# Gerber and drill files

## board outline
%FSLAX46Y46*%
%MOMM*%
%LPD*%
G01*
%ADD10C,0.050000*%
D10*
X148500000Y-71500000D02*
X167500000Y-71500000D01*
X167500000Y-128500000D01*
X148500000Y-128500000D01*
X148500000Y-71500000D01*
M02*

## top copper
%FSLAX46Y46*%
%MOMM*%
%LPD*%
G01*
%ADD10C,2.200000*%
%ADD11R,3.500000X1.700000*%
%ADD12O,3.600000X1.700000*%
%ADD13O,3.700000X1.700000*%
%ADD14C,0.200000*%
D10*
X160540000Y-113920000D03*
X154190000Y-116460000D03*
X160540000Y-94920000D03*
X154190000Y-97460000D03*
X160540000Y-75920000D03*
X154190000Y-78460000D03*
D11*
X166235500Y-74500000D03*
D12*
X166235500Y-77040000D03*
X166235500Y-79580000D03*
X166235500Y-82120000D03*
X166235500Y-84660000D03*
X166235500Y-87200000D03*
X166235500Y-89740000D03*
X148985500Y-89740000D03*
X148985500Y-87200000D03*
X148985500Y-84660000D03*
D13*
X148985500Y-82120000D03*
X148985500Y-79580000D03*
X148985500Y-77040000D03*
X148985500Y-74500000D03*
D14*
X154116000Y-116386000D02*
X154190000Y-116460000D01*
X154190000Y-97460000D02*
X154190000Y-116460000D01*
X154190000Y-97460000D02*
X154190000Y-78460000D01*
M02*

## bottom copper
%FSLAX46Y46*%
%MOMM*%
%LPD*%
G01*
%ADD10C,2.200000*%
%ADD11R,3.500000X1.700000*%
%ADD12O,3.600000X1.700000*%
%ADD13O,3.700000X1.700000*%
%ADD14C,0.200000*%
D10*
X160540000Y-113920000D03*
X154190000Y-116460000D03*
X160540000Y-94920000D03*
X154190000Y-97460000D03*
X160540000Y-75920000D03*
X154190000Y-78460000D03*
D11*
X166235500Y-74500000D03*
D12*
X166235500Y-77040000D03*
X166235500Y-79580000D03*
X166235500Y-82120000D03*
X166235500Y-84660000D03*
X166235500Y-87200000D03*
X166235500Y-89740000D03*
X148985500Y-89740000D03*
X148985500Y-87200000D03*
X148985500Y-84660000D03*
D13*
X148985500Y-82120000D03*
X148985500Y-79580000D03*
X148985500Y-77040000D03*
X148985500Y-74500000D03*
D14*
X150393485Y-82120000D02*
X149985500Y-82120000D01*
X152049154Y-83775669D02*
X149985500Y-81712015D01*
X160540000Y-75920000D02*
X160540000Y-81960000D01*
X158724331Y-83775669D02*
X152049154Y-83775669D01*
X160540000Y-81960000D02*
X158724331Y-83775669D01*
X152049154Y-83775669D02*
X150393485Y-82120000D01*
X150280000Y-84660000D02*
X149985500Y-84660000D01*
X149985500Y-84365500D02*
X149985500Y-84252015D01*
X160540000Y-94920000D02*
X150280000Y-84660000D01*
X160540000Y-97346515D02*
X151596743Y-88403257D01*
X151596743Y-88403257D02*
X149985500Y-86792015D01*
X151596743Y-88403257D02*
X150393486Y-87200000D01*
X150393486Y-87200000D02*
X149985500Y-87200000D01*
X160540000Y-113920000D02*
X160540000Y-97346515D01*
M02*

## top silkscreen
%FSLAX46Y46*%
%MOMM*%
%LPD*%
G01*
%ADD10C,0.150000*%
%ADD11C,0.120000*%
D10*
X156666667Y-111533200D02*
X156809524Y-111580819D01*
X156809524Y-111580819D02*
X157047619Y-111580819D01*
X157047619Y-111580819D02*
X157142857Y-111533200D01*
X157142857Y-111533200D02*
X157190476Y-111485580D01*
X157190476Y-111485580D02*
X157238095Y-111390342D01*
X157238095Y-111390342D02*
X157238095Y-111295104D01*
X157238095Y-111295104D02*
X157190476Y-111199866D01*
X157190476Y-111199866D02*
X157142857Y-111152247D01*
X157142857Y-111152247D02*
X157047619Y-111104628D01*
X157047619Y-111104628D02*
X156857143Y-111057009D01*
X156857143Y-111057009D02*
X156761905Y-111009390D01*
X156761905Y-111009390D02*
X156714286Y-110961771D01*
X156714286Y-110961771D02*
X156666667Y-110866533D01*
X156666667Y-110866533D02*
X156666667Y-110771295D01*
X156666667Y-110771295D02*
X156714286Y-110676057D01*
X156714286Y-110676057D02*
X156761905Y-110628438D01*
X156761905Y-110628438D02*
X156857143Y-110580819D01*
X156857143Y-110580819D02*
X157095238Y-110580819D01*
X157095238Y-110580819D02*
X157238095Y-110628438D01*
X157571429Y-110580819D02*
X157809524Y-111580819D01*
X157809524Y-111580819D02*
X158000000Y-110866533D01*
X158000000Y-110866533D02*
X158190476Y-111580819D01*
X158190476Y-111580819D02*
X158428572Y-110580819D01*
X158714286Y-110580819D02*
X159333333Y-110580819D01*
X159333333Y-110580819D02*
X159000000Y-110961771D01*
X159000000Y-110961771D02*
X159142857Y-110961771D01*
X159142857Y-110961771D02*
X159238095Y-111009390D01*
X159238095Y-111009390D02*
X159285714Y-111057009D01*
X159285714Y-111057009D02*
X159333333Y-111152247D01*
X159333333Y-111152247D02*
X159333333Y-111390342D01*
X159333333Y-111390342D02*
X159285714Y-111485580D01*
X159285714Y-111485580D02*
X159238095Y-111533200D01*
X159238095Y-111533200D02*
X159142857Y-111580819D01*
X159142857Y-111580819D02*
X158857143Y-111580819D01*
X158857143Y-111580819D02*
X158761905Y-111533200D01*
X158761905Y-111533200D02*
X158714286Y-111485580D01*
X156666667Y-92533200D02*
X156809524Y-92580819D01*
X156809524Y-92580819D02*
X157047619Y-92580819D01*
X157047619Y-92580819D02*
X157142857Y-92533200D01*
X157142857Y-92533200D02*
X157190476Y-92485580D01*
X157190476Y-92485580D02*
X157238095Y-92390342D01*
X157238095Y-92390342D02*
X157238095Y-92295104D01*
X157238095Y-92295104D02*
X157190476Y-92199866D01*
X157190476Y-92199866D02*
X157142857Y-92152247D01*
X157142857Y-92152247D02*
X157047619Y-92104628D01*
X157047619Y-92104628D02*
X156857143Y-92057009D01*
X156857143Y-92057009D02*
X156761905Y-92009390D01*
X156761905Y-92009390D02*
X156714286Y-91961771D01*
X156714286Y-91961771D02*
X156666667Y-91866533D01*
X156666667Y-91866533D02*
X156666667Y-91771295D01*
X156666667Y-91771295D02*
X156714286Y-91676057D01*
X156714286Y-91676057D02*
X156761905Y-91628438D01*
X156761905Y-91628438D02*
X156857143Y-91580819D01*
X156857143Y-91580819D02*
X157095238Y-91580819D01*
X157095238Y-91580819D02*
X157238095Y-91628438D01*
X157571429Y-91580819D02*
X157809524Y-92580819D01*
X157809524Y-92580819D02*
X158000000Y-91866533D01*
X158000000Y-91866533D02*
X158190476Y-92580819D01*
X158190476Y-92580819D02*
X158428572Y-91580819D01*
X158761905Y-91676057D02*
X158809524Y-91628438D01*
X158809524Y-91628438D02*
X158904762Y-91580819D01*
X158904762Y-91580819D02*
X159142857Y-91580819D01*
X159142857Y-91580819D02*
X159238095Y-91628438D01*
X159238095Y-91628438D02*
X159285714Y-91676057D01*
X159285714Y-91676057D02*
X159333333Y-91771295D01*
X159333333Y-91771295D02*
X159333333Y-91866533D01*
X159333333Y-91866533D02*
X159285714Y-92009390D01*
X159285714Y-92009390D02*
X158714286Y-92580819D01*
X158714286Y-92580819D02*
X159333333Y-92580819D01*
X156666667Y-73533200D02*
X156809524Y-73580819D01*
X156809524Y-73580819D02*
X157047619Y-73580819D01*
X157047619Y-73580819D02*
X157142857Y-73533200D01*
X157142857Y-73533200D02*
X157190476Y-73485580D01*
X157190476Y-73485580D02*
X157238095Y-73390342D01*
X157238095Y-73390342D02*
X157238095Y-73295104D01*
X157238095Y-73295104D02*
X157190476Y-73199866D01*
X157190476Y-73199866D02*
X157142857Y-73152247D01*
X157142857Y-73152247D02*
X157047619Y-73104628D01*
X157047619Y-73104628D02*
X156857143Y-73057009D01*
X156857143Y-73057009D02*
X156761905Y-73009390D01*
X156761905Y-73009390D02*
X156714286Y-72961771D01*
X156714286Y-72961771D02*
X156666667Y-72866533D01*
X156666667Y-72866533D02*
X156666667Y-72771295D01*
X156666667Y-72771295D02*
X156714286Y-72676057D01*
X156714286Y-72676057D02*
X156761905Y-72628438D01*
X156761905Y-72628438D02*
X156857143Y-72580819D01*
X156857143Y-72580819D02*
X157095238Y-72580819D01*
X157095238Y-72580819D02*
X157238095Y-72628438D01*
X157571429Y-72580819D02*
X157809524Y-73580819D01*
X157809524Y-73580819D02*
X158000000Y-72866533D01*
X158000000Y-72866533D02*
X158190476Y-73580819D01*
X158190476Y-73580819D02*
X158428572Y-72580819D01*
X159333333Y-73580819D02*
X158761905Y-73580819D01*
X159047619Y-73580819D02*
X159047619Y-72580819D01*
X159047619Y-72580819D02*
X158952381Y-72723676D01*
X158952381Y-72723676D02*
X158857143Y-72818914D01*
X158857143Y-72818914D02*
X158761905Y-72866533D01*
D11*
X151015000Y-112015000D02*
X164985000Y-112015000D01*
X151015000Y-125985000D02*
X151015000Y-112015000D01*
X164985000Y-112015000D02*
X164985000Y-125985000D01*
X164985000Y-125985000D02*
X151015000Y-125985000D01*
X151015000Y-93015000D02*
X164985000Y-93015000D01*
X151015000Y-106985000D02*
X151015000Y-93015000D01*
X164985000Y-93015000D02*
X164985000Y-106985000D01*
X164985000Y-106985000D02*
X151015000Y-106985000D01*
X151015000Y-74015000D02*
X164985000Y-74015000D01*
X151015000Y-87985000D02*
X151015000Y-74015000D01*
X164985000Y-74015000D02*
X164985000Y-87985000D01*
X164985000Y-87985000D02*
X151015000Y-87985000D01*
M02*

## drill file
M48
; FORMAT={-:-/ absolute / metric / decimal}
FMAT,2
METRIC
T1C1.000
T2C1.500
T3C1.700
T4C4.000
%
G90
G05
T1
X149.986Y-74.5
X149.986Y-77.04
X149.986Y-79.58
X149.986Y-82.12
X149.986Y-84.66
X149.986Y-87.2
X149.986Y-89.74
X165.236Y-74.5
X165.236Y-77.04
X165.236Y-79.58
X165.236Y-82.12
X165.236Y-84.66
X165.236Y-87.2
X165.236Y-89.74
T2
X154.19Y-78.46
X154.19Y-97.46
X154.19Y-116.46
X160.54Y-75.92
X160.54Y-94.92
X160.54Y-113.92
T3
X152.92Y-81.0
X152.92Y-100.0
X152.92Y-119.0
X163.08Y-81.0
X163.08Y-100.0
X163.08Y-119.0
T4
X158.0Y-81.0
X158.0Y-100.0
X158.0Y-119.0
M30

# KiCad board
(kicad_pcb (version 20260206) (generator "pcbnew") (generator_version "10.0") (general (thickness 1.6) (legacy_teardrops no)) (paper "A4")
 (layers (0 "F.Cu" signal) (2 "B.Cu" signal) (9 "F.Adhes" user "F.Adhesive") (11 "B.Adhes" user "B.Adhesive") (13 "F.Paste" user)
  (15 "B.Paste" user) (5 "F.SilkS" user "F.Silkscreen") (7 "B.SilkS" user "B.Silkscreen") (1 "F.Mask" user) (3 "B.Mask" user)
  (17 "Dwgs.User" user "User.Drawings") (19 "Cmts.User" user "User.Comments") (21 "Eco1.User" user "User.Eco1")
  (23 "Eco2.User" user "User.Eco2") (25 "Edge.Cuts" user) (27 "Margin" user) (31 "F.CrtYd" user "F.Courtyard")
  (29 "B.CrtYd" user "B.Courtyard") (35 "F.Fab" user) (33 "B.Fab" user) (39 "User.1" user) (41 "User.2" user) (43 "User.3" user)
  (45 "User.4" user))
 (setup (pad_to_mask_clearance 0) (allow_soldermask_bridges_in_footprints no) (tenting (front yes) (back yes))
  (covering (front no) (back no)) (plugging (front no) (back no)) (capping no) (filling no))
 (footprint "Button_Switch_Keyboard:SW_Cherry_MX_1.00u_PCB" (layer "F.Cu") (at 160.54 113.92)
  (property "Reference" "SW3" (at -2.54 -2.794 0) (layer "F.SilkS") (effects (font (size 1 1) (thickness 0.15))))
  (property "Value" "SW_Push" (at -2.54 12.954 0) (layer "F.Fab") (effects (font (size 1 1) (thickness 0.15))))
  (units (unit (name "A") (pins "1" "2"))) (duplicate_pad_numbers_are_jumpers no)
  (fp_line (start -9.525 -1.905) (end 4.445 -1.905) (stroke (width 0.12) (type solid)) (layer "F.SilkS"))
  (fp_line (start -9.525 12.065) (end -9.525 -1.905) (stroke (width 0.12) (type solid)) (layer "F.SilkS"))
  (fp_line (start 4.445 -1.905) (end 4.445 12.065) (stroke (width 0.12) (type solid)) (layer "F.SilkS"))
  (fp_line (start 4.445 12.065) (end -9.525 12.065) (stroke (width 0.12) (type solid)) (layer "F.SilkS"))
  (pad "" np_thru_hole circle (at -7.62 5.08) (size 1.7 1.7) (drill 1.7) (layers "*.Cu" "*.Mask"))
  (pad "" np_thru_hole circle (at -2.54 5.08) (size 4 4) (drill 4) (layers "*.Cu" "*.Mask"))
  (pad "" np_thru_hole circle (at 2.54 5.08) (size 1.7 1.7) (drill 1.7) (layers "*.Cu" "*.Mask"))
  (pad "1" thru_hole circle (at 0 0) (size 2.2 2.2) (drill 1.5) (layers "*.Cu" "*.Mask") (remove_unused_layers no)
   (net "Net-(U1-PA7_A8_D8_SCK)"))
  (pad "2" thru_hole circle (at -6.35 2.54) (size 2.2 2.2) (drill 1.5) (layers "*.Cu" "*.Mask") (remove_unused_layers no) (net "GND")))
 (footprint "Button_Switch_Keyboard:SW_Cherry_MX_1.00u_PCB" (layer "F.Cu") (at 160.54 94.92)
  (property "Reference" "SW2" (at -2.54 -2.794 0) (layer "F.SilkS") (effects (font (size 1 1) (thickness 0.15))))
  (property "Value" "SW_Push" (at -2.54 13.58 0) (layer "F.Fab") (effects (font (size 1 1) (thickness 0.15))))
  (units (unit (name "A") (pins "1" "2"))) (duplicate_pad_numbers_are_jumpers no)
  (fp_line (start -9.525 -1.905) (end 4.445 -1.905) (stroke (width 0.12) (type solid)) (layer "F.SilkS"))
  (fp_line (start -9.525 12.065) (end -9.525 -1.905) (stroke (width 0.12) (type solid)) (layer "F.SilkS"))
  (fp_line (start 4.445 -1.905) (end 4.445 12.065) (stroke (width 0.12) (type solid)) (layer "F.SilkS"))
  (fp_line (start 4.445 12.065) (end -9.525 12.065) (stroke (width 0.12) (type solid)) (layer "F.SilkS"))
  (pad "" np_thru_hole circle (at -7.62 5.08) (size 1.7 1.7) (drill 1.7) (layers "*.Cu" "*.Mask"))
  (pad "" np_thru_hole circle (at -2.54 5.08) (size 4 4) (drill 4) (layers "*.Cu" "*.Mask"))
  (pad "" np_thru_hole circle (at 2.54 5.08) (size 1.7 1.7) (drill 1.7) (layers "*.Cu" "*.Mask"))
  (pad "1" thru_hole circle (at 0 0) (size 2.2 2.2) (drill 1.5) (layers "*.Cu" "*.Mask") (remove_unused_layers no)
   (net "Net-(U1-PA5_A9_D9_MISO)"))
  (pad "2" thru_hole circle (at -6.35 2.54) (size 2.2 2.2) (drill 1.5) (layers "*.Cu" "*.Mask") (remove_unused_layers no) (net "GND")))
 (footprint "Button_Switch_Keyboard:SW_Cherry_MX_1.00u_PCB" (layer "F.Cu") (at 160.54 75.92)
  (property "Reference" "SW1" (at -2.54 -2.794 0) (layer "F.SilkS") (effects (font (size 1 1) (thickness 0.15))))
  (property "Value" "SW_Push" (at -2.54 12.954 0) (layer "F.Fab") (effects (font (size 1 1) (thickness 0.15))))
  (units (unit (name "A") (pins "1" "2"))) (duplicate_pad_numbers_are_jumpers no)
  (fp_line (start -9.525 -1.905) (end 4.445 -1.905) (stroke (width 0.12) (type solid)) (layer "F.SilkS"))
  (fp_line (start -9.525 12.065) (end -9.525 -1.905) (stroke (width 0.12) (type solid)) (layer "F.SilkS"))
  (fp_line (start 4.445 -1.905) (end 4.445 12.065) (stroke (width 0.12) (type solid)) (layer "F.SilkS"))
  (fp_line (start 4.445 12.065) (end -9.525 12.065) (stroke (width 0.12) (type solid)) (layer "F.SilkS"))
  (pad "" np_thru_hole circle (at -7.62 5.08) (size 1.7 1.7) (drill 1.7) (layers "*.Cu" "*.Mask"))
  (pad "" np_thru_hole circle (at -2.54 5.08) (size 4 4) (drill 4) (layers "*.Cu" "*.Mask"))
  (pad "" np_thru_hole circle (at 2.54 5.08) (size 1.7 1.7) (drill 1.7) (layers "*.Cu" "*.Mask"))
  (pad "1" thru_hole circle (at 0 0) (size 2.2 2.2) (drill 1.5) (layers "*.Cu" "*.Mask") (remove_unused_layers no)
   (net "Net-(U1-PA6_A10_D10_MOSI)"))
  (pad "2" thru_hole circle (at -6.35 2.54) (size 2.2 2.2) (drill 1.5) (layers "*.Cu" "*.Mask") (remove_unused_layers no) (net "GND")))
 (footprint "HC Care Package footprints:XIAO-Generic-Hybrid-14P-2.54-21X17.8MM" (layer "B.Cu") (at 157.6105 82.12 180)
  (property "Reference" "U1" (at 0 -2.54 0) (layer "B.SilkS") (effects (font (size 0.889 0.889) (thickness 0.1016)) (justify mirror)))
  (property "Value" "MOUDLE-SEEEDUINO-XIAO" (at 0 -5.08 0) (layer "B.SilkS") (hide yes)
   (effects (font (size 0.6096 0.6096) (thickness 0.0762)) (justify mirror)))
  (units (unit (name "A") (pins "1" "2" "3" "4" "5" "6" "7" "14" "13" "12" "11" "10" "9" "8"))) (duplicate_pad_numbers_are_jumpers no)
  (pad "1" thru_hole rect (at -7.625 7.62 180) (size 3.5 1.7) (drill 1 (offset -1 0)) (layers "*.Cu" "*.Mask") (remove_unused_layers no)
   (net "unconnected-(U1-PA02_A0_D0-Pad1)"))
  (pad "2" thru_hole oval (at -7.625 5.08 180) (size 3.6 1.7) (drill 1 (offset -1 0)) (layers "*.Cu" "*.Mask") (remove_unused_layers no)
   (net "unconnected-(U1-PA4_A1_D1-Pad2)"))
  (pad "3" thru_hole oval (at -7.625 2.54 180) (size 3.6 1.7) (drill 1 (offset -1 0)) (layers "*.Cu" "*.Mask") (remove_unused_layers no)
   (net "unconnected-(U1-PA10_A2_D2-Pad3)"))
  (pad "4" thru_hole oval (at -7.625 0 180) (size 3.6 1.7) (drill 1 (offset -1 0)) (layers "*.Cu" "*.Mask") (remove_unused_layers no)
   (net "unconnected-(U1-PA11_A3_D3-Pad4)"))
  (pad "5" thru_hole oval (at -7.625 -2.54 180) (size 3.6 1.7) (drill 1 (offset -1 0)) (layers "*.Cu" "*.Mask") (remove_unused_layers no)
   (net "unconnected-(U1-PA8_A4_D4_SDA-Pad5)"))
  (pad "6" thru_hole oval (at -7.625 -5.08) (size 3.6 1.7) (drill 1 (offset 1 0)) (layers "*.Cu" "*.Mask") (remove_unused_layers no)
   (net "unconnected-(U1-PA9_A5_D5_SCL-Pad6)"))
  (pad "7" thru_hole oval (at -7.625 -7.62 180) (size 3.6 1.7) (drill 1 (offset -1 0)) (layers "*.Cu" "*.Mask") (remove_unused_layers no)
   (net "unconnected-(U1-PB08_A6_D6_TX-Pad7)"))
  (pad "8" thru_hole oval (at 7.625 -7.62 180) (size 3.6 1.7) (drill 1 (offset 1 0)) (layers "*.Cu" "*.Mask") (remove_unused_layers no)
   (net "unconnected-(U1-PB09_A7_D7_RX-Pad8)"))
  (pad "9" thru_hole oval (at 7.625 -5.08 180) (size 3.6 1.7) (drill 1 (offset 1 0)) (layers "*.Cu" "*.Mask") (remove_unused_layers no)
   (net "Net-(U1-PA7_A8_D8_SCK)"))
  (pad "10" thru_hole oval (at 7.625 -2.54 180) (size 3.6 1.7) (drill 1 (offset 1 0)) (layers "*.Cu" "*.Mask") (remove_unused_layers no)
   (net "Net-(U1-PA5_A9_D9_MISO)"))
  (pad "11" thru_hole oval (at 7.625 0 180) (size 3.7 1.7) (drill 1 (offset 1 0)) (layers "*.Cu" "*.Mask") (remove_unused_layers no)
   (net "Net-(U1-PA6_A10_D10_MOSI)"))
  (pad "12" thru_hole oval (at 7.625 2.54 180) (size 3.7 1.7) (drill 1 (offset 1 0)) (layers "*.Cu" "*.Mask") (remove_unused_layers no)
   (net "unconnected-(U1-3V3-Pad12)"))
  (pad "13" thru_hole oval (at 7.625 5.08 180) (size 3.7 1.7) (drill 1 (offset 1 0)) (layers "*.Cu" "*.Mask") (remove_unused_layers no)
   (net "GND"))
  (pad "14" thru_hole oval (at 7.625 7.62 180) (size 3.7 1.7) (drill 1 (offset 1 0)) (layers "*.Cu" "*.Mask") (remove_unused_layers no)
   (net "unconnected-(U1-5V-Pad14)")))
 (gr_rect (start 148.5 71.5) (end 167.5 128.5) (stroke (width 0.05) (type default)) (fill no) (layer "Edge.Cuts"))
 (segment (start 150.393485 82.12) (end 149.9855 82.12) (width 0.2) (layer "B.Cu") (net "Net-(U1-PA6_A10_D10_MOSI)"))
 (segment (start 152.049154 83.775669) (end 149.9855 81.712015) (width 0.2) (layer "B.Cu") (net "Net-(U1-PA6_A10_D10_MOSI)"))
 (segment (start 160.54 75.92) (end 160.54 81.96) (width 0.2) (layer "B.Cu") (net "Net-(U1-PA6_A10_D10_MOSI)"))
 (segment (start 158.724331 83.775669) (end 152.049154 83.775669) (width 0.2) (layer "B.Cu") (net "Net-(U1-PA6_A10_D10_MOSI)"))
 (segment (start 160.54 81.96) (end 158.724331 83.775669) (width 0.2) (layer "B.Cu") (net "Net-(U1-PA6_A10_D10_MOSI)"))
 (segment (start 152.049154 83.775669) (end 150.393485 82.12) (width 0.2) (layer "B.Cu") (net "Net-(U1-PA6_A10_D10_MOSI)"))
 (segment (start 154.116 116.386) (end 154.19 116.46) (width 0.2) (layer "F.Cu") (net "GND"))
 (segment (start 154.19 97.46) (end 154.19 116.46) (width 0.2) (layer "F.Cu") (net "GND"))
 (segment (start 154.19 97.46) (end 154.19 78.46) (width 0.2) (layer "F.Cu") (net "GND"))
 (segment (start 150.28 84.66) (end 149.9855 84.66) (width 0.2) (layer "B.Cu") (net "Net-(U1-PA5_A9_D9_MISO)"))
 (segment (start 149.9855 84.3655) (end 149.9855 84.252015) (width 0.2) (layer "B.Cu") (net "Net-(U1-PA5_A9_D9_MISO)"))
 (segment (start 160.54 94.92) (end 150.28 84.66) (width 0.2) (layer "B.Cu") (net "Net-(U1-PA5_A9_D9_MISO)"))
 (segment (start 160.54 97.346515) (end 151.596743 88.403257) (width 0.2) (layer "B.Cu") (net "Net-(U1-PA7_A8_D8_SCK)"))
 (segment (start 151.596743 88.403257) (end 149.9855 86.792015) (width 0.2) (layer "B.Cu") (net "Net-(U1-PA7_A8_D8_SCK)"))
 (segment (start 151.596743 88.403257) (end 150.393486 87.2) (width 0.2) (layer "B.Cu") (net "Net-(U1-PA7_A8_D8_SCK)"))
 (segment (start 150.393486 87.2) (end 149.9855 87.2) (width 0.2) (layer "B.Cu") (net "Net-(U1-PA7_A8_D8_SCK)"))
 (segment (start 160.54 113.92) (end 160.54 97.346515) (width 0.2) (layer "B.Cu") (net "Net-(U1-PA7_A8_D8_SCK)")))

